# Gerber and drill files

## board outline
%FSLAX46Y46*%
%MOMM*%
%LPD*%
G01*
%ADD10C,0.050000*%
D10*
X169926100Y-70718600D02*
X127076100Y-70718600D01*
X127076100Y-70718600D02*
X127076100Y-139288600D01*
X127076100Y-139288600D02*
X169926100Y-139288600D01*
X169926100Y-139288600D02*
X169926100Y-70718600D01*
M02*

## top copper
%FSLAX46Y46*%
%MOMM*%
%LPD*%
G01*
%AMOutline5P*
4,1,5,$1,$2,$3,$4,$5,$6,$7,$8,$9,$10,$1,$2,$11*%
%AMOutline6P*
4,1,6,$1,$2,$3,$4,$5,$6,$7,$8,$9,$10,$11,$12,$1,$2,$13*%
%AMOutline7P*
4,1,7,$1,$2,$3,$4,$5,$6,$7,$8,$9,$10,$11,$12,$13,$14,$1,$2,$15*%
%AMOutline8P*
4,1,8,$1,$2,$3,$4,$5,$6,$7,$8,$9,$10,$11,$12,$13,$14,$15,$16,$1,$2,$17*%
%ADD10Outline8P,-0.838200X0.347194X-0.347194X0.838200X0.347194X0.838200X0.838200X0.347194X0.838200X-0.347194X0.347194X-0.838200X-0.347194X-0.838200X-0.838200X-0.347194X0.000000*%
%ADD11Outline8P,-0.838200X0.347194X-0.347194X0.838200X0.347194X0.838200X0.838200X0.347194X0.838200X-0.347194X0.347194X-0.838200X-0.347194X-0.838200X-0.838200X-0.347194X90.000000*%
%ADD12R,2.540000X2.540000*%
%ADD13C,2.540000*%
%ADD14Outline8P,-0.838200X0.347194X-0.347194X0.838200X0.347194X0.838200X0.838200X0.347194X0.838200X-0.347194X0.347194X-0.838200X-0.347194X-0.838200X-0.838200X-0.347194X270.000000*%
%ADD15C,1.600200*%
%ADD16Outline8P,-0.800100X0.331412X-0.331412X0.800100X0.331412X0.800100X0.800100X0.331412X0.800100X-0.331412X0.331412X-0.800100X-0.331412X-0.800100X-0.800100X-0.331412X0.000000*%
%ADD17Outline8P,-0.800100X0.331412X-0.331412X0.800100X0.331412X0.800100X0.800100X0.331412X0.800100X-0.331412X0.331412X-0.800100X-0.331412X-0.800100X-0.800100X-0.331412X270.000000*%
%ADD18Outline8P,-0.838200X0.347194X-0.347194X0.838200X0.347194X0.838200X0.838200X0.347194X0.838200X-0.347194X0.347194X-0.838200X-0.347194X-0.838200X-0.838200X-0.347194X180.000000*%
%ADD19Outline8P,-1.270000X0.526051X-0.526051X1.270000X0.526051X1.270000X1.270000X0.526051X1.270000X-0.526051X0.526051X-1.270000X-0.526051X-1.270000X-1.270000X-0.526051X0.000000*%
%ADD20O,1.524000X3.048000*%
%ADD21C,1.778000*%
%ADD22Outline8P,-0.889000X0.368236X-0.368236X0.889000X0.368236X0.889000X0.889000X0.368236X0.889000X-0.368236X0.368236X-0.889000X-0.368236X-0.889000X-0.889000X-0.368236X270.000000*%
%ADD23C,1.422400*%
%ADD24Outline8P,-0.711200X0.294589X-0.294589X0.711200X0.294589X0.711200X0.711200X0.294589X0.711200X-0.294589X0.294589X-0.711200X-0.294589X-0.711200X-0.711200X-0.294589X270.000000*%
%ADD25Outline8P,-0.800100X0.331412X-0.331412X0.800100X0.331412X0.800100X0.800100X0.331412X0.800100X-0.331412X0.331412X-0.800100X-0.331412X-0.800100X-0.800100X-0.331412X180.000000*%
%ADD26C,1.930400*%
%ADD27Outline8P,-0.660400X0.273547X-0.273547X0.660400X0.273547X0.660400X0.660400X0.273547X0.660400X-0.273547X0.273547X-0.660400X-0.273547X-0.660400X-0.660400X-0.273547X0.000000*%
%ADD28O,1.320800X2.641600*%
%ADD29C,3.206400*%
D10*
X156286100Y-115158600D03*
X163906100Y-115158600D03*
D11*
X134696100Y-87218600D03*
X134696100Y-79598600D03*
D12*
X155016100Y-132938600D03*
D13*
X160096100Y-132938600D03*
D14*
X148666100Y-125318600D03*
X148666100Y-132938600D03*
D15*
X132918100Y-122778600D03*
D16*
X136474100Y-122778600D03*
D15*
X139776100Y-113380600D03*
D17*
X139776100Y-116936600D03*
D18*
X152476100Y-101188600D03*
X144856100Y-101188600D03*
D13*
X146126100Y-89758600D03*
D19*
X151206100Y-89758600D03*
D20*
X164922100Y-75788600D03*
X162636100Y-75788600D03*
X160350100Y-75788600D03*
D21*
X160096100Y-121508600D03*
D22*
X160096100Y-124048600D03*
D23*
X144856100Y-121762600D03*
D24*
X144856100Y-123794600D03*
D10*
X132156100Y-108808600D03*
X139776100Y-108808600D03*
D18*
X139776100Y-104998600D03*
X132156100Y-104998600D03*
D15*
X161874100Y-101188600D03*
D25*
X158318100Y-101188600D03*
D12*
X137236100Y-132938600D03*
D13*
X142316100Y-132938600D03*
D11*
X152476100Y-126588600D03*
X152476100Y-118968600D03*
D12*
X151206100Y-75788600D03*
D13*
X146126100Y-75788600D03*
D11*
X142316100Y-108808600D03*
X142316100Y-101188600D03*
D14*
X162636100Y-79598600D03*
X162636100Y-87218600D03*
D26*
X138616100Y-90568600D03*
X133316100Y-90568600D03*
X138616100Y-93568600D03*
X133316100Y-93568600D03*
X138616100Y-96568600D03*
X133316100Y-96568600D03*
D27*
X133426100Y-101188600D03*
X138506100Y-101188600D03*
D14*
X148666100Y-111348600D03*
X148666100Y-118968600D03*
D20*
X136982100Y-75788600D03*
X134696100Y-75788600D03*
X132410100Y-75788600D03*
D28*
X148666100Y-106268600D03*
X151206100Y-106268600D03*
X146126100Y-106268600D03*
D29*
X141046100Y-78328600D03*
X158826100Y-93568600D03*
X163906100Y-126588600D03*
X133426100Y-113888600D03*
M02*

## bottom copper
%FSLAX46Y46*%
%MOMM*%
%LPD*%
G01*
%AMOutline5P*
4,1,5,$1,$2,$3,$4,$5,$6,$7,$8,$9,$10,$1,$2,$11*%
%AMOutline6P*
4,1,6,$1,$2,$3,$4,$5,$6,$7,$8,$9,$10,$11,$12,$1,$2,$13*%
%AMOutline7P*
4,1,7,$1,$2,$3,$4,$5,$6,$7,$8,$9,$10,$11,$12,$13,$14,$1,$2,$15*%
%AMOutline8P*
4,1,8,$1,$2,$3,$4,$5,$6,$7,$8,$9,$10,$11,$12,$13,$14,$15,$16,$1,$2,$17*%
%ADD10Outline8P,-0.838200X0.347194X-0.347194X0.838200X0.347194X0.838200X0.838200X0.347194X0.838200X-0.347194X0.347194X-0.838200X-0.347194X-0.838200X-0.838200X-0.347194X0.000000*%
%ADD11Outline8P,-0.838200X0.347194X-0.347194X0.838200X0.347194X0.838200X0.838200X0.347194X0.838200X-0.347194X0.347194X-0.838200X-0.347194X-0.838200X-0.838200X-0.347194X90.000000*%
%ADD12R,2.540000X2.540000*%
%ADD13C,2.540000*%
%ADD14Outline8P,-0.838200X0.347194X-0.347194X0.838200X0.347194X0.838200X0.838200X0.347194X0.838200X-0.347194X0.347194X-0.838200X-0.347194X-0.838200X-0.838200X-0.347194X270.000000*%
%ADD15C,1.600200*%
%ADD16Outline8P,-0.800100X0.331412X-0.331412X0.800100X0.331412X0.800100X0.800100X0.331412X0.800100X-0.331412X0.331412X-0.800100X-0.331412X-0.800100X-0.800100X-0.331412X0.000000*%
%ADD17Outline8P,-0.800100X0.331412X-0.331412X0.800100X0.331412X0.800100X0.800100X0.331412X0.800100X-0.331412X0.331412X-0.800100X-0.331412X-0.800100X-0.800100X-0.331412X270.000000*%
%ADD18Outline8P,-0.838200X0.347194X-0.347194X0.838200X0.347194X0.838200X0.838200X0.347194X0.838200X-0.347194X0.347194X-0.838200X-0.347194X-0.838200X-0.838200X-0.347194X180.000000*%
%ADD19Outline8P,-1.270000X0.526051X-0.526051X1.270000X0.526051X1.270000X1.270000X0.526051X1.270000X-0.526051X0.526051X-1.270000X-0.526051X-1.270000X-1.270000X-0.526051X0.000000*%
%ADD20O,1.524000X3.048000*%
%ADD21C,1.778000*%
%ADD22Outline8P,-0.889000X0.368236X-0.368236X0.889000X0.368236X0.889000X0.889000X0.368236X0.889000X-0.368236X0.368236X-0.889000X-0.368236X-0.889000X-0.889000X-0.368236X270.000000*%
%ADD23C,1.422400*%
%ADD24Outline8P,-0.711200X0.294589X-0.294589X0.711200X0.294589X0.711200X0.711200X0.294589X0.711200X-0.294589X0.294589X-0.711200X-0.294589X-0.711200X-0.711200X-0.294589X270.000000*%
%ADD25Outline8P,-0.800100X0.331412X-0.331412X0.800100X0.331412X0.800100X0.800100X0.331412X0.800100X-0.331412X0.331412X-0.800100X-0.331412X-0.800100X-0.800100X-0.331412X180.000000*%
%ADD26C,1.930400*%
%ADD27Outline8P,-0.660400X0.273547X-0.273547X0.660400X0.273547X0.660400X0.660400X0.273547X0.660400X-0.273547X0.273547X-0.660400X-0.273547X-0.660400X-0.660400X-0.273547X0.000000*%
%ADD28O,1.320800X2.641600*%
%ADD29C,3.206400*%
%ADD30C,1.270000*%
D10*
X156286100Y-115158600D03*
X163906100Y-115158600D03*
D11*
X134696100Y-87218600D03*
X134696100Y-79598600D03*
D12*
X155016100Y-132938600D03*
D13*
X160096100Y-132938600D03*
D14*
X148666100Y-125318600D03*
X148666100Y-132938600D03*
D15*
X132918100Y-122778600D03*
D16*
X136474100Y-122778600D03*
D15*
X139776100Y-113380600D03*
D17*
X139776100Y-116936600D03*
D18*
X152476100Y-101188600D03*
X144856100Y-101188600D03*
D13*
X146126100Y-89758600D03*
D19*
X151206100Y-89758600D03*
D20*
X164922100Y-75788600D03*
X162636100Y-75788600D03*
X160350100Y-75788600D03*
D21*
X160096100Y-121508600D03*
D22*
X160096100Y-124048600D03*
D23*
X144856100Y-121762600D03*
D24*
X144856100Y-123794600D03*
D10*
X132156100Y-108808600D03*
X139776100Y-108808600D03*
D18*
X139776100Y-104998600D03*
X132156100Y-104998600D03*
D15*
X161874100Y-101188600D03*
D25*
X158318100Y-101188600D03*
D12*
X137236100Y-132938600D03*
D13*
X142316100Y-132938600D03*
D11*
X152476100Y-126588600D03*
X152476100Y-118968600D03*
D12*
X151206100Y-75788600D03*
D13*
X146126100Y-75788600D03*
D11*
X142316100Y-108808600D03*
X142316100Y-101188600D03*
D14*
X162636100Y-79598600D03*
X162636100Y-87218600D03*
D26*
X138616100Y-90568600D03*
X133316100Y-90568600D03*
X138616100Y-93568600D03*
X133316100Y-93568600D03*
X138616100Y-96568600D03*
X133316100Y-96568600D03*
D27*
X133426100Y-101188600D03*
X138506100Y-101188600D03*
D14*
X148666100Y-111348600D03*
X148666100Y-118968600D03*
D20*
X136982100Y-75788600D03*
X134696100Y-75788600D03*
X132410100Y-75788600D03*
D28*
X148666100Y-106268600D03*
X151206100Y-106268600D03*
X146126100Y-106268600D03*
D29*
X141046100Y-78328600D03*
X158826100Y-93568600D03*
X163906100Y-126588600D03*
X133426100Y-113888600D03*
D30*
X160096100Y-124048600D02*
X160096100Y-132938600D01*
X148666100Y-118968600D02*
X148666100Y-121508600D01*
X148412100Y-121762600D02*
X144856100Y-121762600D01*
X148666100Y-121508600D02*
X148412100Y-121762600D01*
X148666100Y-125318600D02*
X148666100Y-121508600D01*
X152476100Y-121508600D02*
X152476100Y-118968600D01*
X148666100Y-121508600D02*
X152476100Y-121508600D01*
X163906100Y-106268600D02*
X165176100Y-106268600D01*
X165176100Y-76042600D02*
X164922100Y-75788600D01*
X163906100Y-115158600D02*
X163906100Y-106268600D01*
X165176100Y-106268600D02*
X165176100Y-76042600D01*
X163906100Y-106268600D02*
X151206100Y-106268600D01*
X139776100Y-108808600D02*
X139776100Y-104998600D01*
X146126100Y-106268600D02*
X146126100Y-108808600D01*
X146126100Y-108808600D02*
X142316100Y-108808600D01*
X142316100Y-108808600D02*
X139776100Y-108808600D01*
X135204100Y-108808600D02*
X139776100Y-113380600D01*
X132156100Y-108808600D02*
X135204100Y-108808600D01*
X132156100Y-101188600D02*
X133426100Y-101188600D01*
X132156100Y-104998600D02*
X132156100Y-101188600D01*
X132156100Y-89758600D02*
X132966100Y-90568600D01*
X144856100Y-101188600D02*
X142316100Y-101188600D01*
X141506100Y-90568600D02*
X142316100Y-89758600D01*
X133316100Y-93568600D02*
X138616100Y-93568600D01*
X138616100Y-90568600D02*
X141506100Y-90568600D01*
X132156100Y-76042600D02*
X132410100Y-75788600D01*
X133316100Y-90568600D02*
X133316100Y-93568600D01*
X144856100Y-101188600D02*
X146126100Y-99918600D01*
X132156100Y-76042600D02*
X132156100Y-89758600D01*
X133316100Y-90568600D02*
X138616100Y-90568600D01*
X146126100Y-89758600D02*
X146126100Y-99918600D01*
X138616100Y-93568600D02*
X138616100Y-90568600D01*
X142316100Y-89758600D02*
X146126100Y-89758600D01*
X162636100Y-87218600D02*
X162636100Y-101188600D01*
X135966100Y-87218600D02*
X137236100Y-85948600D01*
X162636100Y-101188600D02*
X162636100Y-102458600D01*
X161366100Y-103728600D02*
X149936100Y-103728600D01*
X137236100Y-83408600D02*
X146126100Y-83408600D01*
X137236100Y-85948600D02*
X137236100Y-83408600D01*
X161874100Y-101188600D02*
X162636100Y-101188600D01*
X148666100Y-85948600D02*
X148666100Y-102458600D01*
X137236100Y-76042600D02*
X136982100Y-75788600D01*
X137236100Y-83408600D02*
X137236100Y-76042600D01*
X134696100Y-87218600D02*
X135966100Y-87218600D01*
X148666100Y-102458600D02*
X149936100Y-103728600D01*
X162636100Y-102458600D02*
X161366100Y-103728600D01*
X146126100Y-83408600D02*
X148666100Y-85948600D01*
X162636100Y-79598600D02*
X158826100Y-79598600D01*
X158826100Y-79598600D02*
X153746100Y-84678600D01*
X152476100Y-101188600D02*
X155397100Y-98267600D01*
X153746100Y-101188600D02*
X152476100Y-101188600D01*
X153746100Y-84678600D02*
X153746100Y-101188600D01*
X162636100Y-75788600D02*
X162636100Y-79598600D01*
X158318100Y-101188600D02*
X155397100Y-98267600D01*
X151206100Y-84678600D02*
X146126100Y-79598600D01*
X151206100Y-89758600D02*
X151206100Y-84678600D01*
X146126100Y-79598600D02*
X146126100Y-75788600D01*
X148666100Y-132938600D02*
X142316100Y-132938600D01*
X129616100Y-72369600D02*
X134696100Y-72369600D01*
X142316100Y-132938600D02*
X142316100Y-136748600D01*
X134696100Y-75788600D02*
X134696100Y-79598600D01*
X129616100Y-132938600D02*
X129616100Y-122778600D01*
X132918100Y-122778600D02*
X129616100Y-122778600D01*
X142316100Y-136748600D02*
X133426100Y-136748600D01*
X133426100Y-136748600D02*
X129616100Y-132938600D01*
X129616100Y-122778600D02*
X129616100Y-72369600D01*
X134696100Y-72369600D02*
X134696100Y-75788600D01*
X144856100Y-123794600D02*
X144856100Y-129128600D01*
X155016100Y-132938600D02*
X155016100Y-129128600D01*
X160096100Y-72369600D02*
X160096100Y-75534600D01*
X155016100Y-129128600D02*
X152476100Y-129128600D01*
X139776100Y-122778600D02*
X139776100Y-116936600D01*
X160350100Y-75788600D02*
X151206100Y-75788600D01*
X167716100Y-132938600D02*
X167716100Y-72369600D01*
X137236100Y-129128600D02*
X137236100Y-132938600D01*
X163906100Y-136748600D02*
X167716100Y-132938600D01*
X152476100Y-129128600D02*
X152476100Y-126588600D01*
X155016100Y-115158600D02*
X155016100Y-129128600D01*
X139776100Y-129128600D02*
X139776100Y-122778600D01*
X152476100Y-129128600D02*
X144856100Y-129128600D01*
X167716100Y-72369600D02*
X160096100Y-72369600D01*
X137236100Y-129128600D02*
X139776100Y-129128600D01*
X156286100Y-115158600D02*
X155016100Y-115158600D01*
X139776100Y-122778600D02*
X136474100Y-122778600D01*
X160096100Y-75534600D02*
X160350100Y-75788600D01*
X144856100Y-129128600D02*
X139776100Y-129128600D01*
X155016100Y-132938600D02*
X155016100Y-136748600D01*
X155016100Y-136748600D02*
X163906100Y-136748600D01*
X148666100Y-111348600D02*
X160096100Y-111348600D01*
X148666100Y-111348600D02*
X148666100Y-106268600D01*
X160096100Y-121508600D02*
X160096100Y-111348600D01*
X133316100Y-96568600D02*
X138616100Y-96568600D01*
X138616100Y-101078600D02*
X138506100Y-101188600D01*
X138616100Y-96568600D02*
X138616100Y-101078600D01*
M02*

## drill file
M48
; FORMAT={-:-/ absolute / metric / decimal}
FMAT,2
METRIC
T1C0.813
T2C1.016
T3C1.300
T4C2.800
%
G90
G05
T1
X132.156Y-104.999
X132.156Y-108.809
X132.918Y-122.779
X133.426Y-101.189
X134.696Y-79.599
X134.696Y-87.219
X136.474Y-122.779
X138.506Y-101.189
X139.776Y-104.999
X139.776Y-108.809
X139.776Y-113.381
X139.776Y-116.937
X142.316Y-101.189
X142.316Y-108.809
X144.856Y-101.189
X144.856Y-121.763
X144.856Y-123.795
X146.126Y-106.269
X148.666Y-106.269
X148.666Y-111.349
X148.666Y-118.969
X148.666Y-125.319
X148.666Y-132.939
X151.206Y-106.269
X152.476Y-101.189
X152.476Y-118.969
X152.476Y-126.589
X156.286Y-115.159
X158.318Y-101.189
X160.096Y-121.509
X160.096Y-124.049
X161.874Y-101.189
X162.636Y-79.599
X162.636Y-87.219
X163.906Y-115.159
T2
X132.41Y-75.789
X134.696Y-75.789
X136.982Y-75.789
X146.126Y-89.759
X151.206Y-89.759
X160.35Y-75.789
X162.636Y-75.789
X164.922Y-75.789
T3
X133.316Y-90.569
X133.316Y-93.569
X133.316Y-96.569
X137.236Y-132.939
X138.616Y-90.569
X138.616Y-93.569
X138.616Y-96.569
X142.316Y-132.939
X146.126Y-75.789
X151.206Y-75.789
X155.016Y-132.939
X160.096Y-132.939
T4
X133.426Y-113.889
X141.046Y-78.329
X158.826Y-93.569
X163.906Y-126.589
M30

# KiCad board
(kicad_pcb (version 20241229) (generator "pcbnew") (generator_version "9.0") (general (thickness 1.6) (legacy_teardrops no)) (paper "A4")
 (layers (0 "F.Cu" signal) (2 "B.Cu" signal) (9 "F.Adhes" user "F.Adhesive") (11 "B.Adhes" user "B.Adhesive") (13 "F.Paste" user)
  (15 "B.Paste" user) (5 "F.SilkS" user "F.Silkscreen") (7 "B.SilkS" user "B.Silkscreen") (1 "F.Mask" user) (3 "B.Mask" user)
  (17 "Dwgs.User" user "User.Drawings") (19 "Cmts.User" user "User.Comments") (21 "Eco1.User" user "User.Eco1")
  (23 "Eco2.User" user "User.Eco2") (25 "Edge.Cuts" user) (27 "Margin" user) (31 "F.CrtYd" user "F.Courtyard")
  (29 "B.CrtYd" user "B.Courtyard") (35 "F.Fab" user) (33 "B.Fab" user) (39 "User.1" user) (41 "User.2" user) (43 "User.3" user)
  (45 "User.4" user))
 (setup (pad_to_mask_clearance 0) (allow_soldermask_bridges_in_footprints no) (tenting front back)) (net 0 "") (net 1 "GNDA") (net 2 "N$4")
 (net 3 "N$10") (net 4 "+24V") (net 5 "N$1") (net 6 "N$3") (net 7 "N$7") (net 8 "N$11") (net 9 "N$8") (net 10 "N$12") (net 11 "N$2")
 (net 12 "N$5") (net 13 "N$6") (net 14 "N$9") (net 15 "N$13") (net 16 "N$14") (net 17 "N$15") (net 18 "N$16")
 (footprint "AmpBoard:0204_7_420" (layer "F.Cu") (at 160.0961 115.1586)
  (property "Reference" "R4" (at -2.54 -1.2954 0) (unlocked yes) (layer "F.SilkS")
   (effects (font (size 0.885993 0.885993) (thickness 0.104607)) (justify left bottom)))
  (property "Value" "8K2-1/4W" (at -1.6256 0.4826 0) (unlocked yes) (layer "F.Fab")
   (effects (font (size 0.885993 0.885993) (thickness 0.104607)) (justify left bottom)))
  (pad "1" thru_hole roundrect (at -3.81 0) (size 1.6764 1.6764) (drill 0.8128) (layers "*.Cu" "*.Mask") (remove_unused_layers no)
   (roundrect_rratio 0.25) (chamfer_ratio 0.2928932188) (chamfer top_left top_right bottom_left bottom_right) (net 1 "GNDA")
   (solder_mask_margin 0.1016) (thermal_bridge_angle 0))
  (pad "2" thru_hole roundrect (at 3.81 0) (size 1.6764 1.6764) (drill 0.8128) (layers "*.Cu" "*.Mask") (remove_unused_layers no)
   (roundrect_rratio 0.25) (chamfer_ratio 0.2928932188) (chamfer top_left top_right bottom_left bottom_right) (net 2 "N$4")
   (solder_mask_margin 0.1016) (thermal_bridge_angle 0)))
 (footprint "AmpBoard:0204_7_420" (layer "F.Cu") (at 134.6961 83.4086 90)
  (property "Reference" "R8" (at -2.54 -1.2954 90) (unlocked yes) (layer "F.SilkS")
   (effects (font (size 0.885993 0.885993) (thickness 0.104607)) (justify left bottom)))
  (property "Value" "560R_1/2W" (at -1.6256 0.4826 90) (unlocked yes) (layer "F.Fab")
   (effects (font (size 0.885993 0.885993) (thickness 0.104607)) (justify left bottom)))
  (pad "1" thru_hole roundrect (at -3.81 0 90) (size 1.6764 1.6764) (drill 0.8128) (layers "*.Cu" "*.Mask") (remove_unused_layers no)
   (roundrect_rratio 0.25) (chamfer_ratio 0.2928932188) (chamfer top_left top_right bottom_left bottom_right) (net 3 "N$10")
   (solder_mask_margin 0.1016) (thermal_bridge_angle 0))
  (pad "2" thru_hole roundrect (at 3.81 0 90) (size 1.6764 1.6764) (drill 0.8128) (layers "*.Cu" "*.Mask") (remove_unused_layers no)
   (roundrect_rratio 0.25) (chamfer_ratio 0.2928932188) (chamfer top_left top_right bottom_left bottom_right) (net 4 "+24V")
   (solder_mask_margin 0.1016) (thermal_bridge_angle 0)))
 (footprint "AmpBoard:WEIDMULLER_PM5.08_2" (layer "F.Cu") (at 157.5561 132.9386)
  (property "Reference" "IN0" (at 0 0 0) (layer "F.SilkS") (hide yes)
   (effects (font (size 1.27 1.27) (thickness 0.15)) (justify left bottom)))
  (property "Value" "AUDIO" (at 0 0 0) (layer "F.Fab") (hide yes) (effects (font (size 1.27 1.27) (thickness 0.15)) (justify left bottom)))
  (pad "1" thru_hole rect (at -2.54 0) (size 2.54 2.54) (drill 1.3) (layers "*.Cu" "*.Mask") (remove_unused_layers no) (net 1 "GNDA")
   (solder_mask_margin 0.1016) (thermal_bridge_angle 0))
  (pad "2" thru_hole circle (at 2.54 0) (size 2.54 2.54) (drill 1.3) (layers "*.Cu" "*.Mask") (remove_unused_layers no) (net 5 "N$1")
   (solder_mask_margin 0.1016) (thermal_bridge_angle 0)))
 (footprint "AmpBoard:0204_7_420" (layer "F.Cu") (at 148.6661 129.1286 -90)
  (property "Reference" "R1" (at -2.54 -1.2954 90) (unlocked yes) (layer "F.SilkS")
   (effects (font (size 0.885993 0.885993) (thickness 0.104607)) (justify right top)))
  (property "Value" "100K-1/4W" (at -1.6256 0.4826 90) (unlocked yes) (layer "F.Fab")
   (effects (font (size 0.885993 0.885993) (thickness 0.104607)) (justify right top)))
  (pad "1" thru_hole roundrect (at -3.81 0 270) (size 1.6764 1.6764) (drill 0.8128) (layers "*.Cu" "*.Mask") (remove_unused_layers no)
   (roundrect_rratio 0.25) (chamfer_ratio 0.2928932188) (chamfer top_left top_right bottom_left bottom_right) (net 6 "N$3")
   (solder_mask_margin 0.1016) (thermal_bridge_angle 0))
  (pad "2" thru_hole roundrect (at 3.81 0 270) (size 1.6764 1.6764) (drill 0.8128) (layers "*.Cu" "*.Mask") (remove_unused_layers no)
   (roundrect_rratio 0.25) (chamfer_ratio 0.2928932188) (chamfer top_left top_right bottom_left bottom_right) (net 4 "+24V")
   (solder_mask_margin 0.1016) (thermal_bridge_angle 0)))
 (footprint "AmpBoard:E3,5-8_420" (layer "F.Cu") (at 134.6961 122.7786)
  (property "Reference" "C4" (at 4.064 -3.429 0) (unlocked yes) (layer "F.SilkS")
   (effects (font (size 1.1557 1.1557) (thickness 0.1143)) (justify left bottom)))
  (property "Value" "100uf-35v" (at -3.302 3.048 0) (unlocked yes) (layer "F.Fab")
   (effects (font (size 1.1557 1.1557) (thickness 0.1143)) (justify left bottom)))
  (pad "+" thru_hole circle (at -1.778 0) (size 1.6002 1.6002) (drill 0.8128) (layers "*.Cu" "*.Mask") (remove_unused_layers no)
   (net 4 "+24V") (solder_mask_margin 0.1016) (thermal_bridge_angle 0))
  (pad "-" thru_hole roundrect (at 1.778 0) (size 1.6002 1.6002) (drill 0.8128) (layers "*.Cu" "*.Mask") (remove_unused_layers no)
   (roundrect_rratio 0.25) (chamfer_ratio 0.2928932188) (chamfer top_left top_right bottom_left bottom_right) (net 1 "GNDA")
   (solder_mask_margin 0.1016) (thermal_bridge_angle 0)))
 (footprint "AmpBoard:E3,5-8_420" (layer "F.Cu") (at 139.7761 115.1586 -90)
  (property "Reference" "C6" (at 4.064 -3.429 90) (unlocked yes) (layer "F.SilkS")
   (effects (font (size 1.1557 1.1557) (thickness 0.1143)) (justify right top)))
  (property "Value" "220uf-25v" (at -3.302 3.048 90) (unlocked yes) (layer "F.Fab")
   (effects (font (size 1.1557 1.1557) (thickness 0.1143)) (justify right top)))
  (pad "+" thru_hole circle (at -1.778 0 270) (size 1.6002 1.6002) (drill 0.8128) (layers "*.Cu" "*.Mask") (remove_unused_layers no)
   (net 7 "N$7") (solder_mask_margin 0.1016) (thermal_bridge_angle 0))
  (pad "-" thru_hole roundrect (at 1.778 0 270) (size 1.6002 1.6002) (drill 0.8128) (layers "*.Cu" "*.Mask") (remove_unused_layers no)
   (roundrect_rratio 0.25) (chamfer_ratio 0.2928932188) (chamfer top_left top_right bottom_left bottom_right) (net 1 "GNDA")
   (solder_mask_margin 0.1016) (thermal_bridge_angle 0)))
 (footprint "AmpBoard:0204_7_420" (layer "F.Cu") (at 148.6661 101.1886 180)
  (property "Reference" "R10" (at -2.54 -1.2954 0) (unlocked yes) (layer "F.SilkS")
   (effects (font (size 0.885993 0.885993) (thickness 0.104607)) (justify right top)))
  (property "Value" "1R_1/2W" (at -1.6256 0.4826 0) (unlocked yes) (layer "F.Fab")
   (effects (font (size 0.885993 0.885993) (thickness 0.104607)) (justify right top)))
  (pad "1" thru_hole roundrect (at -3.81 0 180) (size 1.6764 1.6764) (drill 0.8128) (layers "*.Cu" "*.Mask") (remove_unused_layers no)
   (roundrect_rratio 0.25) (chamfer_ratio 0.2928932188) (chamfer top_left top_right bottom_left bottom_right) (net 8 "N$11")
   (solder_mask_margin 0.1016) (thermal_bridge_angle 0))
  (pad "2" thru_hole roundrect (at 3.81 0 180) (size 1.6764 1.6764) (drill 0.8128) (layers "*.Cu" "*.Mask") (remove_unused_layers no)
   (roundrect_rratio 0.25) (chamfer_ratio 0.2928932188) (chamfer top_left top_right bottom_left bottom_right) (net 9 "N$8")
   (solder_mask_margin 0.1016) (thermal_bridge_angle 0)))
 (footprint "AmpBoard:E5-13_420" (layer "F.Cu") (at 148.6661 89.7586)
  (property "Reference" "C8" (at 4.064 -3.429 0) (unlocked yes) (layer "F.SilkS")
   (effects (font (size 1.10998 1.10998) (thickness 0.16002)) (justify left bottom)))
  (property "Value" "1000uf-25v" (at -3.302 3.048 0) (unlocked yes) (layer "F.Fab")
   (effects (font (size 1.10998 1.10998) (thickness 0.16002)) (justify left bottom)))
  (pad "+" thru_hole circle (at -2.54 0) (size 2.54 2.54) (drill 1.016) (layers "*.Cu" "*.Mask") (remove_unused_layers no) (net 9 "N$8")
   (solder_mask_margin 0.1016) (thermal_bridge_angle 0))
  (pad "-" thru_hole roundrect (at 2.54 0) (size 2.54 2.54) (drill 1.016) (layers "*.Cu" "*.Mask") (remove_unused_layers no)
   (roundrect_rratio 0.25) (chamfer_ratio 0.2928932188) (chamfer top_left top_right bottom_left bottom_right) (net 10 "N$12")
   (solder_mask_margin 0.1016) (thermal_bridge_angle 0)))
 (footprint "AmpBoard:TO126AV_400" (layer "F.Cu") (at 162.6361 74.5186)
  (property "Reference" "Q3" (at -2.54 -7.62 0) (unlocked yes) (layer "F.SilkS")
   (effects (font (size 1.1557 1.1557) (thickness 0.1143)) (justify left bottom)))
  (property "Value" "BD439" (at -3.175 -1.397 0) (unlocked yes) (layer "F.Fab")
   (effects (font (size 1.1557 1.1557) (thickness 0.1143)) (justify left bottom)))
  (pad "B" thru_hole oval (at 2.286 1.27 90) (size 3.048 1.524) (drill 1.016) (layers "*.Cu" "*.Mask") (remove_unused_layers no)
   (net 2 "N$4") (solder_mask_margin 0.1016) (thermal_bridge_angle 0))
  (pad "C" thru_hole oval (at 0 1.27 90) (size 3.048 1.524) (drill 1.016) (layers "*.Cu" "*.Mask") (remove_unused_layers no) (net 8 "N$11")
   (solder_mask_margin 0.1016) (thermal_bridge_angle 0))
  (pad "E" thru_hole oval (at -2.286 1.27 90) (size 3.048 1.524) (drill 1.016) (layers "*.Cu" "*.Mask") (remove_unused_layers no)
   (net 1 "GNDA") (solder_mask_margin 0.1016) (thermal_bridge_angle 0)))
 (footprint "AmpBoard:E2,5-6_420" (layer "F.Cu") (at 160.0961 122.7786 -90)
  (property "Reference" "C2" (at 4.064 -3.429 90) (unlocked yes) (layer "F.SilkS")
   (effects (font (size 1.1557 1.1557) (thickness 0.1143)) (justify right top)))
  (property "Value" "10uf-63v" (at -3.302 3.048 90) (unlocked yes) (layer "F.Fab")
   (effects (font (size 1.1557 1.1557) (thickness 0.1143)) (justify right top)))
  (pad "+" thru_hole circle (at -1.27 0 270) (size 1.778 1.778) (drill 0.8128) (layers "*.Cu" "*.Mask") (remove_unused_layers no)
   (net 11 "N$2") (solder_mask_margin 0.1016) (thermal_bridge_angle 0))
  (pad "-" thru_hole roundrect (at 1.27 0 270) (size 1.778 1.778) (drill 0.8128) (layers "*.Cu" "*.Mask") (remove_unused_layers no)
   (roundrect_rratio 0.25) (chamfer_ratio 0.2928932188) (chamfer top_left top_right bottom_left bottom_right) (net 5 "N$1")
   (solder_mask_margin 0.1016) (thermal_bridge_angle 0)))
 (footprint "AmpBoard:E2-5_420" (layer "F.Cu") (at 144.8561 122.7786 -90)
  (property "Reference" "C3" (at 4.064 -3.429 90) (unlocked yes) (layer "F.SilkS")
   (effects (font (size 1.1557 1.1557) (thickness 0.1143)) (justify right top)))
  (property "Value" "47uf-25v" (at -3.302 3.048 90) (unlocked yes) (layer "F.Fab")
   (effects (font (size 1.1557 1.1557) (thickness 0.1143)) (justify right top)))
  (pad "+" thru_hole circle (at -1.016 0 270) (size 1.4224 1.4224) (drill 0.8128) (layers "*.Cu" "*.Mask") (remove_unused_layers no)
   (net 6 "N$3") (solder_mask_margin 0.1016) (thermal_bridge_angle 0))
  (pad "-" thru_hole roundrect (at 1.016 0 270) (size 1.4224 1.4224) (drill 0.8128) (layers "*.Cu" "*.Mask") (remove_unused_layers no)
   (roundrect_rratio 0.25) (chamfer_ratio 0.2928932188) (chamfer top_left top_right bottom_left bottom_right) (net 1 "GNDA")
   (solder_mask_margin 0.1016) (thermal_bridge_angle 0)))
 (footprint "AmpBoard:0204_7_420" (layer "F.Cu") (at 135.9661 108.8086)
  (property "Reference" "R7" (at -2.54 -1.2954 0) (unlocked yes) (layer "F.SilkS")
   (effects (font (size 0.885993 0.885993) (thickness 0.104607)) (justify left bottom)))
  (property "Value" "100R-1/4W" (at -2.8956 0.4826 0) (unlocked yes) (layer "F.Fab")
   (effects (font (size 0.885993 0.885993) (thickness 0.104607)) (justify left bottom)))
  (pad "1" thru_hole roundrect (at -3.81 0) (size 1.6764 1.6764) (drill 0.8128) (layers "*.Cu" "*.Mask") (remove_unused_layers no)
   (roundrect_rratio 0.25) (chamfer_ratio 0.2928932188) (chamfer top_left top_right bottom_left bottom_right) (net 7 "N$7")
   (solder_mask_margin 0.1016) (thermal_bridge_angle 0))
  (pad "2" thru_hole roundrect (at 3.81 0) (size 1.6764 1.6764) (drill 0.8128) (layers "*.Cu" "*.Mask") (remove_unused_layers no)
   (roundrect_rratio 0.25) (chamfer_ratio 0.2928932188) (chamfer top_left top_right bottom_left bottom_right) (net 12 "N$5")
   (solder_mask_margin 0.1016) (thermal_bridge_angle 0)))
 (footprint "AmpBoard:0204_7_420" (layer "F.Cu") (at 135.9661 104.9986 180)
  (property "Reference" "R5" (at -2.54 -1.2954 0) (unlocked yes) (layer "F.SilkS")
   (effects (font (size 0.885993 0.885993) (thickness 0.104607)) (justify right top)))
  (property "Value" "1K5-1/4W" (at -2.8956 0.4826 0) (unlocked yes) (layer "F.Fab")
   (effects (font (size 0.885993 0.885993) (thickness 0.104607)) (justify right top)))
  (pad "1" thru_hole roundrect (at -3.81 0 180) (size 1.6764 1.6764) (drill 0.8128) (layers "*.Cu" "*.Mask") (remove_unused_layers no)
   (roundrect_rratio 0.25) (chamfer_ratio 0.2928932188) (chamfer top_left top_right bottom_left bottom_right) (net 12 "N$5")
   (solder_mask_margin 0.1016) (thermal_bridge_angle 0))
  (pad "2" thru_hole roundrect (at 3.81 0 180) (size 1.6764 1.6764) (drill 0.8128) (layers "*.Cu" "*.Mask") (remove_unused_layers no)
   (roundrect_rratio 0.25) (chamfer_ratio 0.2928932188) (chamfer top_left top_right bottom_left bottom_right) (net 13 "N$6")
   (solder_mask_margin 0.1016) (thermal_bridge_angle 0)))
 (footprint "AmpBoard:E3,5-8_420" (layer "F.Cu") (at 160.0961 101.1886 180)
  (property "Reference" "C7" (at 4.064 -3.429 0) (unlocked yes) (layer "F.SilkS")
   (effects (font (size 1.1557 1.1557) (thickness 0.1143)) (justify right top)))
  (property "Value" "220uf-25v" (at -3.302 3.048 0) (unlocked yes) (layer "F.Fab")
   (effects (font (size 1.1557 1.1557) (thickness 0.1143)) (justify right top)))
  (pad "+" thru_hole circle (at -1.778 0 180) (size 1.6002 1.6002) (drill 0.8128) (layers "*.Cu" "*.Mask") (remove_unused_layers no)
   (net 3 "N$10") (solder_mask_margin 0.1016) (thermal_bridge_angle 0))
  (pad "-" thru_hole roundrect (at 1.778 0 180) (size 1.6002 1.6002) (drill 0.8128) (layers "*.Cu" "*.Mask") (remove_unused_layers no)
   (roundrect_rratio 0.25) (chamfer_ratio 0.2928932188) (chamfer top_left top_right bottom_left bottom_right) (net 8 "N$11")
   (solder_mask_margin 0.1016) (thermal_bridge_angle 0)))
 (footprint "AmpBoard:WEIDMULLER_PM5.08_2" (layer "F.Cu") (at 139.7761 132.9386)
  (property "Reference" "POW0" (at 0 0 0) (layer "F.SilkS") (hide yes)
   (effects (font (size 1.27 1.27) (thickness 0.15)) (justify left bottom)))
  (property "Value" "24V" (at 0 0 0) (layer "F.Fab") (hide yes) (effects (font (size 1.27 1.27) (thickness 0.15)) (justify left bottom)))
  (pad "1" thru_hole rect (at -2.54 0) (size 2.54 2.54) (drill 1.3) (layers "*.Cu" "*.Mask") (remove_unused_layers no) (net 1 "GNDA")
   (solder_mask_margin 0.1016) (thermal_bridge_angle 0))
  (pad "2" thru_hole circle (at 2.54 0) (size 2.54 2.54) (drill 1.3) (layers "*.Cu" "*.Mask") (remove_unused_layers no) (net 4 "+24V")
   (solder_mask_margin 0.1016) (thermal_bridge_angle 0)))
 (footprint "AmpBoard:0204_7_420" (layer "F.Cu") (at 152.4761 122.7786 90)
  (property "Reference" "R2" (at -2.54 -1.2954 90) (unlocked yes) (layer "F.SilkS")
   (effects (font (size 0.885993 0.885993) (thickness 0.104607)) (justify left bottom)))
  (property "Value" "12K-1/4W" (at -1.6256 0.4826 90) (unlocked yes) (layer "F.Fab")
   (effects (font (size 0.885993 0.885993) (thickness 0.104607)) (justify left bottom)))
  (pad "1" thru_hole roundrect (at -3.81 0 90) (size 1.6764 1.6764) (drill 0.8128) (layers "*.Cu" "*.Mask") (remove_unused_layers no)
   (roundrect_rratio 0.25) (chamfer_ratio 0.2928932188) (chamfer top_left top_right bottom_left bottom_right) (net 1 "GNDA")
   (solder_mask_margin 0.1016) (thermal_bridge_angle 0))
  (pad "2" thru_hole roundrect (at 3.81 0 90) (size 1.6764 1.6764) (drill 0.8128) (layers "*.Cu" "*.Mask") (remove_unused_layers no)
   (roundrect_rratio 0.25) (chamfer_ratio 0.2928932188) (chamfer top_left top_right bottom_left bottom_right) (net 6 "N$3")
   (solder_mask_margin 0.1016) (thermal_bridge_angle 0)))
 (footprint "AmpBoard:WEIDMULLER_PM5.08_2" (layer "F.Cu") (at 148.6661 75.7886 180)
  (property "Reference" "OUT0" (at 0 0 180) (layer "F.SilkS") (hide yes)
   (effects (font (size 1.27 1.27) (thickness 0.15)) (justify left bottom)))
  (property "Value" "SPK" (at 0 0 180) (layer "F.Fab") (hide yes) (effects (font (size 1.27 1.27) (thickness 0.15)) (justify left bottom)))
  (pad "1" thru_hole rect (at -2.54 0 180) (size 2.54 2.54) (drill 1.3) (layers "*.Cu" "*.Mask") (remove_unused_layers no) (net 1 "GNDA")
   (solder_mask_margin 0.1016) (thermal_bridge_angle 0))
  (pad "2" thru_hole circle (at 2.54 0 180) (size 2.54 2.54) (drill 1.3) (layers "*.Cu" "*.Mask") (remove_unused_layers no) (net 10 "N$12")
   (solder_mask_margin 0.1016) (thermal_bridge_angle 0)))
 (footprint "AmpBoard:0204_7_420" (layer "F.Cu") (at 142.3161 104.9986 90)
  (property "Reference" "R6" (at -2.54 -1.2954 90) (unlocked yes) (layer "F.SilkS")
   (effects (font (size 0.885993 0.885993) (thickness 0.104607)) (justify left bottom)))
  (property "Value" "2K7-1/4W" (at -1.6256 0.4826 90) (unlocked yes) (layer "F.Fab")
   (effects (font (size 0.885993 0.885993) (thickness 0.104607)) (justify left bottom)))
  (pad "1" thru_hole roundrect (at -3.81 0 90) (size 1.6764 1.6764) (drill 0.8128) (layers "*.Cu" "*.Mask") (remove_unused_layers no)
   (roundrect_rratio 0.25) (chamfer_ratio 0.2928932188) (chamfer top_left top_right bottom_left bottom_right) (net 12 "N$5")
   (solder_mask_margin 0.1016) (thermal_bridge_angle 0))
  (pad "2" thru_hole roundrect (at 3.81 0 90) (size 1.6764 1.6764) (drill 0.8128) (layers "*.Cu" "*.Mask") (remove_unused_layers no)
   (roundrect_rratio 0.25) (chamfer_ratio 0.2928932188) (chamfer top_left top_right bottom_left bottom_right) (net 9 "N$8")
   (solder_mask_margin 0.1016) (thermal_bridge_angle 0)))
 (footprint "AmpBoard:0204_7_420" (layer "F.Cu") (at 162.6361 83.4086 -90)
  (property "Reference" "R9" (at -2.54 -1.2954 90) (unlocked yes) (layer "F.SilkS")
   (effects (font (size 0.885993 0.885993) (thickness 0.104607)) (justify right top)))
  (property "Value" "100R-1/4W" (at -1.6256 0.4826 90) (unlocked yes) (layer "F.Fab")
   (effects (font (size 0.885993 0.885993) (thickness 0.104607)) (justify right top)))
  (pad "1" thru_hole roundrect (at -3.81 0 270) (size 1.6764 1.6764) (drill 0.8128) (layers "*.Cu" "*.Mask") (remove_unused_layers no)
   (roundrect_rratio 0.25) (chamfer_ratio 0.2928932188) (chamfer top_left top_right bottom_left bottom_right) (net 8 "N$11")
   (solder_mask_margin 0.1016) (thermal_bridge_angle 0))
  (pad "2" thru_hole roundrect (at 3.81 0 270) (size 1.6764 1.6764) (drill 0.8128) (layers "*.Cu" "*.Mask") (remove_unused_layers no)
   (roundrect_rratio 0.25) (chamfer_ratio 0.2928932188) (chamfer top_left top_right bottom_left bottom_right) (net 3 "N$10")
   (solder_mask_margin 0.1016) (thermal_bridge_angle 0)))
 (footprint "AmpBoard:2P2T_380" (layer "F.Cu") (at 135.9661 93.5686 -90)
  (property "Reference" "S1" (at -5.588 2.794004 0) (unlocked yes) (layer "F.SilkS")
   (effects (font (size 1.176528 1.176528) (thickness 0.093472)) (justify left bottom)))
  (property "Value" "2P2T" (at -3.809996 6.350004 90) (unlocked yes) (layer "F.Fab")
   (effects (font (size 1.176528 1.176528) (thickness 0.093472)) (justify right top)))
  (pad "1.1" thru_hole circle (at -3 -2.65 270) (size 1.9304 1.9304) (drill 1.3) (layers "*.Cu" "*.Mask") (remove_unused_layers no)
   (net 9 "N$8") (solder_mask_margin 0.1016) (thermal_bridge_angle 0))
  (pad "1.2" thru_hole circle (at -3 2.65 270) (size 1.9304 1.9304) (drill 1.3) (layers "*.Cu" "*.Mask") (remove_unused_layers no)
   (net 9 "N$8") (solder_mask_margin 0.1016) (thermal_bridge_angle 0))
  (pad "2.1" thru_hole circle (at 0 -2.65 270) (size 1.9304 1.9304) (drill 1.3) (layers "*.Cu" "*.Mask") (remove_unused_layers no)
   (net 9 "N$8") (solder_mask_margin 0.1016) (thermal_bridge_angle 0))
  (pad "2.2" thru_hole circle (at 0 2.65 270) (size 1.9304 1.9304) (drill 1.3) (layers "*.Cu" "*.Mask") (remove_unused_layers no)
   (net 9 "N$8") (solder_mask_margin 0.1016) (thermal_bridge_angle 0))
  (pad "3.1" thru_hole circle (at 3 -2.65 270) (size 1.9304 1.9304) (drill 1.3) (layers "*.Cu" "*.Mask") (remove_unused_layers no)
   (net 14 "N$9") (solder_mask_margin 0.1016) (thermal_bridge_angle 0))
  (pad "3.2" thru_hole circle (at 3 2.65 270) (size 1.9304 1.9304) (drill 1.3) (layers "*.Cu" "*.Mask") (remove_unused_layers no)
   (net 14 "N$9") (solder_mask_margin 0.1016) (thermal_bridge_angle 0)))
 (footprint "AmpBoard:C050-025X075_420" (layer "F.Cu") (at 135.9661 101.1886)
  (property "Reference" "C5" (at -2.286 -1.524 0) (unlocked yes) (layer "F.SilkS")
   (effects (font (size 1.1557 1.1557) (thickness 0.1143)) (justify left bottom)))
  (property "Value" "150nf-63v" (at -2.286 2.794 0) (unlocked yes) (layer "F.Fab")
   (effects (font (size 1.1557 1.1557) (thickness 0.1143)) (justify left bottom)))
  (pad "1" thru_hole roundrect (at -2.54 0) (size 1.3208 1.3208) (drill 0.8128) (layers "*.Cu" "*.Mask") (remove_unused_layers no)
   (roundrect_rratio 0.25) (chamfer_ratio 0.2928932188) (chamfer top_left top_right bottom_left bottom_right) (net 13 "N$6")
   (solder_mask_margin 0.1016) (thermal_bridge_angle 0))
  (pad "2" thru_hole roundrect (at 2.54 0) (size 1.3208 1.3208) (drill 0.8128) (layers "*.Cu" "*.Mask") (remove_unused_layers no)
   (roundrect_rratio 0.25) (chamfer_ratio 0.2928932188) (chamfer top_left top_right bottom_left bottom_right) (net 14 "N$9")
   (solder_mask_margin 0.1016) (thermal_bridge_angle 0)))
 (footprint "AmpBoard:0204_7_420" (layer "F.Cu") (at 148.6661 115.1586 -90)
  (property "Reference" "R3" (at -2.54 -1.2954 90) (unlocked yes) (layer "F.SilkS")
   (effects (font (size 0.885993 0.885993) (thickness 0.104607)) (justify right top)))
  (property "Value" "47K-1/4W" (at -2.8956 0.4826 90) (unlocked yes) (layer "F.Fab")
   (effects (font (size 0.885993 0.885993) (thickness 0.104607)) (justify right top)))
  (pad "1" thru_hole roundrect (at -3.81 0 270) (size 1.6764 1.6764) (drill 0.8128) (layers "*.Cu" "*.Mask") (remove_unused_layers no)
   (roundrect_rratio 0.25) (chamfer_ratio 0.2928932188) (chamfer top_left top_right bottom_left bottom_right) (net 11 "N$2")
   (solder_mask_margin 0.1016) (thermal_bridge_angle 0))
  (pad "2" thru_hole roundrect (at 3.81 0 270) (size 1.6764 1.6764) (drill 0.8128) (layers "*.Cu" "*.Mask") (remove_unused_layers no)
   (roundrect_rratio 0.25) (chamfer_ratio 0.2928932188) (chamfer top_left top_right bottom_left bottom_right) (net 6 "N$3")
   (solder_mask_margin 0.1016) (thermal_bridge_angle 0)))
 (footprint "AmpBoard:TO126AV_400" (layer "F.Cu") (at 134.6961 74.5186)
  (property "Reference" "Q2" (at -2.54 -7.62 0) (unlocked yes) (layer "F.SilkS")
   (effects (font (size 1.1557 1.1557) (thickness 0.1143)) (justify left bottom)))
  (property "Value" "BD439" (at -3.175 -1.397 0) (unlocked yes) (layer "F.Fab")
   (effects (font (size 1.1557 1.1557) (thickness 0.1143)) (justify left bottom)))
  (pad "B" thru_hole oval (at 2.286 1.27 90) (size 3.048 1.524) (drill 1.016) (layers "*.Cu" "*.Mask") (remove_unused_layers no)
   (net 3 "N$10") (solder_mask_margin 0.1016) (thermal_bridge_angle 0))
  (pad "C" thru_hole oval (at 0 1.27 90) (size 3.048 1.524) (drill 1.016) (layers "*.Cu" "*.Mask") (remove_unused_layers no) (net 4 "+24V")
   (solder_mask_margin 0.1016) (thermal_bridge_angle 0))
  (pad "E" thru_hole oval (at -2.286 1.27 90) (size 3.048 1.524) (drill 1.016) (layers "*.Cu" "*.Mask") (remove_unused_layers no)
   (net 9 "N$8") (solder_mask_margin 0.1016) (thermal_bridge_angle 0)))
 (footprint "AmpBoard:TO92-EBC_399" (layer "F.Cu") (at 148.6661 107.5386 180)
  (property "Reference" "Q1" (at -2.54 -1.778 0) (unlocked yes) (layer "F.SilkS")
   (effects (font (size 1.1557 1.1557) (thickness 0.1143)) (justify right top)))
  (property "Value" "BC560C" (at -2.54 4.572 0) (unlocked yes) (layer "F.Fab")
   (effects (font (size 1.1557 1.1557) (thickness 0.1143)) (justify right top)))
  (pad "B" thru_hole oval (at 0 1.27 270) (size 2.6416 1.3208) (drill 0.8128) (layers "*.Cu" "*.Mask") (remove_unused_layers no)
   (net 11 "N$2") (solder_mask_margin 0.1016) (thermal_bridge_angle 0))
  (pad "C" thru_hole oval (at -2.54 1.27 270) (size 2.6416 1.3208) (drill 0.8128) (layers "*.Cu" "*.Mask") (remove_unused_layers no)
   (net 2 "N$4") (solder_mask_margin 0.1016) (thermal_bridge_angle 0))
  (pad "E" thru_hole oval (at 2.54 1.27 270) (size 2.6416 1.3208) (drill 0.8128) (layers "*.Cu" "*.Mask") (remove_unused_layers no)
   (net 12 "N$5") (solder_mask_margin 0.1016) (thermal_bridge_angle 0)))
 (gr_line (start 169.9261 70.7186) (end 127.0761 70.7186) (stroke (width 0.05) (type solid)) (layer "Edge.Cuts"))
 (gr_line (start 127.0761 70.7186) (end 127.0761 139.2886) (stroke (width 0.05) (type solid)) (layer "Edge.Cuts"))
 (gr_line (start 127.0761 139.2886) (end 169.9261 139.2886) (stroke (width 0.05) (type solid)) (layer "Edge.Cuts"))
 (gr_line (start 169.9261 139.2886) (end 169.9261 70.7186) (stroke (width 0.05) (type solid)) (layer "Edge.Cuts"))
 (segment (start 160.0961 124.0486) (end 160.0961 132.9386) (width 1.27) (layer "B.Cu") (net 5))
 (segment (start 148.6661 118.9686) (end 148.6661 121.5086) (width 1.27) (layer "B.Cu") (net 6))
 (segment (start 148.4121 121.7626) (end 144.8561 121.7626) (width 1.27) (layer "B.Cu") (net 6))
 (segment (start 148.6661 121.5086) (end 148.4121 121.7626) (width 1.27) (layer "B.Cu") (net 6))
 (segment (start 148.6661 125.3186) (end 148.6661 121.5086) (width 1.27) (layer "B.Cu") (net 6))
 (segment (start 152.4761 121.5086) (end 152.4761 118.9686) (width 1.27) (layer "B.Cu") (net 6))
 (segment (start 148.6661 121.5086) (end 152.4761 121.5086) (width 1.27) (layer "B.Cu") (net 6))
 (segment (start 163.9061 106.2686) (end 165.1761 106.2686) (width 1.27) (layer "B.Cu") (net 2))
 (segment (start 165.1761 76.0426) (end 164.9221 75.7886) (width 1.27) (layer "B.Cu") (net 2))
 (segment (start 163.9061 115.1586) (end 163.9061 106.2686) (width 1.27) (layer "B.Cu") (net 2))
 (segment (start 165.1761 106.2686) (end 165.1761 76.0426) (width 1.27) (layer "B.Cu") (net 2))
 (segment (start 163.9061 106.2686) (end 151.2061 106.2686) (width 1.27) (layer "B.Cu") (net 2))
 (segment (start 139.7761 108.8086) (end 139.7761 104.9986) (width 1.27) (layer "B.Cu") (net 12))
 (segment (start 146.1261 106.2686) (end 146.1261 108.8086) (width 1.27) (layer "B.Cu") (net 12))
 (segment (start 146.1261 108.8086) (end 142.3161 108.8086) (width 1.27) (layer "B.Cu") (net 12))
 (segment (start 142.3161 108.8086) (end 139.7761 108.8086) (width 1.27) (layer "B.Cu") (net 12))
 (segment (start 135.2041 108.8086) (end 139.7761 113.3806) (width 1.27) (layer "B.Cu") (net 7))
 (segment (start 132.1561 108.8086) (end 135.2041 108.8086) (width 1.27) (layer "B.Cu") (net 7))
 (segment (start 132.1561 101.1886) (end 133.4261 101.1886) (width 1.27) (layer "B.Cu") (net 13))
 (segment (start 132.1561 104.9986) (end 132.1561 101.1886) (width 1.27) (layer "B.Cu") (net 13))
 (segment (start 132.1561 89.7586) (end 132.9661 90.5686) (width 1.27) (layer "B.Cu") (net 9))
 (segment (start 144.8561 101.1886) (end 142.3161 101.1886) (width 1.27) (layer "B.Cu") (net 9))
 (segment (start 141.5061 90.5686) (end 142.3161 89.7586) (width 1.27) (layer "B.Cu") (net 9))
 (segment (start 133.3161 93.5686) (end 138.6161 93.5686) (width 1.27) (layer "B.Cu") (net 9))
 (segment (start 138.6161 90.5686) (end 141.5061 90.5686) (width 1.27) (layer "B.Cu") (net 9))
 (segment (start 132.1561 76.0426) (end 132.4101 75.7886) (width 1.27) (layer "B.Cu") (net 9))
 (segment (start 133.3161 90.5686) (end 133.3161 93.5686) (width 1.27) (layer "B.Cu") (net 9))
 (segment (start 144.8561 101.1886) (end 146.1261 99.9186) (width 1.27) (layer "B.Cu") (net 9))
 (segment (start 132.1561 76.0426) (end 132.1561 89.7586) (width 1.27) (layer "B.Cu") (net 9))
 (segment (start 133.3161 90.5686) (end 138.6161 90.5686) (width 1.27) (layer "B.Cu") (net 9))
 (segment (start 146.1261 89.7586) (end 146.1261 99.9186) (width 1.27) (layer "B.Cu") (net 9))
 (segment (start 138.6161 93.5686) (end 138.6161 90.5686) (width 1.27) (layer "B.Cu") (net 9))
 (segment (start 142.3161 89.7586) (end 146.1261 89.7586) (width 1.27) (layer "B.Cu") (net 9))
 (segment (start 162.6361 87.2186) (end 162.6361 101.1886) (width 1.27) (layer "B.Cu") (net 3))
 (segment (start 135.9661 87.2186) (end 137.2361 85.9486) (width 1.27) (layer "B.Cu") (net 3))
 (segment (start 162.6361 101.1886) (end 162.6361 102.4586) (width 1.27) (layer "B.Cu") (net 3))
 (segment (start 161.3661 103.7286) (end 149.9361 103.7286) (width 1.27) (layer "B.Cu") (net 3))
 (segment (start 137.2361 83.4086) (end 146.1261 83.4086) (width 1.27) (layer "B.Cu") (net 3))
 (segment (start 137.2361 85.9486) (end 137.2361 83.4086) (width 1.27) (layer "B.Cu") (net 3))
 (segment (start 161.8741 101.1886) (end 162.6361 101.1886) (width 1.27) (layer "B.Cu") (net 3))
 (segment (start 148.6661 85.9486) (end 148.6661 102.4586) (width 1.27) (layer "B.Cu") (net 3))
 (segment (start 137.2361 76.0426) (end 136.9821 75.7886) (width 1.27) (layer "B.Cu") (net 3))
 (segment (start 137.2361 83.4086) (end 137.2361 76.0426) (width 1.27) (layer "B.Cu") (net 3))
 (segment (start 134.6961 87.2186) (end 135.9661 87.2186) (width 1.27) (layer "B.Cu") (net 3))
 (segment (start 148.6661 102.4586) (end 149.9361 103.7286) (width 1.27) (layer "B.Cu") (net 3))
 (segment (start 162.6361 102.4586) (end 161.3661 103.7286) (width 1.27) (layer "B.Cu") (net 3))
 (segment (start 146.1261 83.4086) (end 148.6661 85.9486) (width 1.27) (layer "B.Cu") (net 3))
 (segment (start 162.6361 79.5986) (end 158.8261 79.5986) (width 1.27) (layer "B.Cu") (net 8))
 (segment (start 158.8261 79.5986) (end 153.7461 84.6786) (width 1.27) (layer "B.Cu") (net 8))
 (segment (start 152.4761 101.1886) (end 155.3971 98.2676) (width 1.27) (layer "B.Cu") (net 8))
 (segment (start 153.7461 101.1886) (end 152.4761 101.1886) (width 1.27) (layer "B.Cu") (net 8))
 (segment (start 153.7461 84.6786) (end 153.7461 101.1886) (width 1.27) (layer "B.Cu") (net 8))
 (segment (start 162.6361 75.7886) (end 162.6361 79.5986) (width 1.27) (layer "B.Cu") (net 8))
 (segment (start 158.3181 101.1886) (end 155.3971 98.2676) (width 1.27) (layer "B.Cu") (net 8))
 (segment (start 151.2061 84.6786) (end 146.1261 79.5986) (width 1.27) (layer "B.Cu") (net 10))
 (segment (start 151.2061 89.7586) (end 151.2061 84.6786) (width 1.27) (layer "B.Cu") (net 10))
 (segment (start 146.1261 79.5986) (end 146.1261 75.7886) (width 1.27) (layer "B.Cu") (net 10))
 (segment (start 148.6661 132.9386) (end 142.3161 132.9386) (width 1.27) (layer "B.Cu") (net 4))
 (segment (start 129.6161 72.3696) (end 134.6961 72.3696) (width 1.27) (layer "B.Cu") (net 4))
 (segment (start 142.3161 132.9386) (end 142.3161 136.7486) (width 1.27) (layer "B.Cu") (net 4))
 (segment (start 134.6961 75.7886) (end 134.6961 79.5986) (width 1.27) (layer "B.Cu") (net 4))
 (segment (start 129.6161 132.9386) (end 129.6161 122.7786) (width 1.27) (layer "B.Cu") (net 4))
 (segment (start 132.9181 122.7786) (end 129.6161 122.7786) (width 1.27) (layer "B.Cu") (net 4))
 (segment (start 142.3161 136.7486) (end 133.4261 136.7486) (width 1.27) (layer "B.Cu") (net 4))
 (segment (start 133.4261 136.7486) (end 129.6161 132.9386) (width 1.27) (layer "B.Cu") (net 4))
 (segment (start 129.6161 122.7786) (end 129.6161 72.3696) (width 1.27) (layer "B.Cu") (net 4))
 (segment (start 134.6961 72.3696) (end 134.6961 75.7886) (width 1.27) (layer "B.Cu") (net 4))
 (segment (start 144.8561 123.7946) (end 144.8561 129.1286) (width 1.27) (layer "B.Cu") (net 1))
 (segment (start 155.0161 132.9386) (end 155.0161 129.1286) (width 1.27) (layer "B.Cu") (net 1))
 (segment (start 160.0961 72.3696) (end 160.0961 75.5346) (width 1.27) (layer "B.Cu") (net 1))
 (segment (start 155.0161 129.1286) (end 152.4761 129.1286) (width 1.27) (layer "B.Cu") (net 1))
 (segment (start 139.7761 122.7786) (end 139.7761 116.9366) (width 1.27) (layer "B.Cu") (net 1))
 (segment (start 160.3501 75.7886) (end 151.2061 75.7886) (width 1.27) (layer "B.Cu") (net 1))
 (segment (start 167.7161 132.9386) (end 167.7161 72.3696) (width 1.27) (layer "B.Cu") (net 1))
 (segment (start 137.2361 129.1286) (end 137.2361 132.9386) (width 1.27) (layer "B.Cu") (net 1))
 (segment (start 163.9061 136.7486) (end 167.7161 132.9386) (width 1.27) (layer "B.Cu") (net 1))
 (segment (start 152.4761 129.1286) (end 152.4761 126.5886) (width 1.27) (layer "B.Cu") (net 1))
 (segment (start 155.0161 115.1586) (end 155.0161 129.1286) (width 1.27) (layer "B.Cu") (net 1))
 (segment (start 139.7761 129.1286) (end 139.7761 122.7786) (width 1.27) (layer "B.Cu") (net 1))
 (segment (start 152.4761 129.1286) (end 144.8561 129.1286) (width 1.27) (layer "B.Cu") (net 1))
 (segment (start 167.7161 72.3696) (end 160.0961 72.3696) (width 1.27) (layer "B.Cu") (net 1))
 (segment (start 137.2361 129.1286) (end 139.7761 129.1286) (width 1.27) (layer "B.Cu") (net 1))
 (segment (start 156.2861 115.1586) (end 155.0161 115.1586) (width 1.27) (layer "B.Cu") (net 1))
 (segment (start 139.7761 122.7786) (end 136.4741 122.7786) (width 1.27) (layer "B.Cu") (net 1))
 (segment (start 160.0961 75.5346) (end 160.3501 75.7886) (width 1.27) (layer "B.Cu") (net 1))
 (segment (start 144.8561 129.1286) (end 139.7761 129.1286) (width 1.27) (layer "B.Cu") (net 1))
 (segment (start 155.0161 132.9386) (end 155.0161 136.7486) (width 1.27) (layer "B.Cu") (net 1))
 (segment (start 155.0161 136.7486) (end 163.9061 136.7486) (width 1.27) (layer "B.Cu") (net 1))
 (segment (start 148.6661 111.3486) (end 160.0961 111.3486) (width 1.27) (layer "B.Cu") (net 11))
 (segment (start 148.6661 111.3486) (end 148.6661 106.2686) (width 1.27) (layer "B.Cu") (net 11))
 (segment (start 160.0961 121.5086) (end 160.0961 111.3486) (width 1.27) (layer "B.Cu") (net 11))
 (segment (start 133.3161 96.5686) (end 138.6161 96.5686) (width 1.27) (layer "B.Cu") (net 14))
 (segment (start 138.6161 101.0786) (end 138.5061 101.1886) (width 1.27) (layer "B.Cu") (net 14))
 (segment (start 138.6161 96.5686) (end 138.6161 101.0786) (width 1.27) (layer "B.Cu") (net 14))
 (via (at 141.0461 78.3286) (size 3.2064) (drill 2.8) (layers "F.Cu" "B.Cu") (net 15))
 (via (at 158.8261 93.5686) (size 3.2064) (drill 2.8) (layers "F.Cu" "B.Cu") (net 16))
 (via (at 163.9061 126.5886) (size 3.2064) (drill 2.8) (layers "F.Cu" "B.Cu") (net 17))
 (via (at 133.4261 113.8886) (size 3.2064) (drill 2.8) (layers "F.Cu" "B.Cu") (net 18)))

